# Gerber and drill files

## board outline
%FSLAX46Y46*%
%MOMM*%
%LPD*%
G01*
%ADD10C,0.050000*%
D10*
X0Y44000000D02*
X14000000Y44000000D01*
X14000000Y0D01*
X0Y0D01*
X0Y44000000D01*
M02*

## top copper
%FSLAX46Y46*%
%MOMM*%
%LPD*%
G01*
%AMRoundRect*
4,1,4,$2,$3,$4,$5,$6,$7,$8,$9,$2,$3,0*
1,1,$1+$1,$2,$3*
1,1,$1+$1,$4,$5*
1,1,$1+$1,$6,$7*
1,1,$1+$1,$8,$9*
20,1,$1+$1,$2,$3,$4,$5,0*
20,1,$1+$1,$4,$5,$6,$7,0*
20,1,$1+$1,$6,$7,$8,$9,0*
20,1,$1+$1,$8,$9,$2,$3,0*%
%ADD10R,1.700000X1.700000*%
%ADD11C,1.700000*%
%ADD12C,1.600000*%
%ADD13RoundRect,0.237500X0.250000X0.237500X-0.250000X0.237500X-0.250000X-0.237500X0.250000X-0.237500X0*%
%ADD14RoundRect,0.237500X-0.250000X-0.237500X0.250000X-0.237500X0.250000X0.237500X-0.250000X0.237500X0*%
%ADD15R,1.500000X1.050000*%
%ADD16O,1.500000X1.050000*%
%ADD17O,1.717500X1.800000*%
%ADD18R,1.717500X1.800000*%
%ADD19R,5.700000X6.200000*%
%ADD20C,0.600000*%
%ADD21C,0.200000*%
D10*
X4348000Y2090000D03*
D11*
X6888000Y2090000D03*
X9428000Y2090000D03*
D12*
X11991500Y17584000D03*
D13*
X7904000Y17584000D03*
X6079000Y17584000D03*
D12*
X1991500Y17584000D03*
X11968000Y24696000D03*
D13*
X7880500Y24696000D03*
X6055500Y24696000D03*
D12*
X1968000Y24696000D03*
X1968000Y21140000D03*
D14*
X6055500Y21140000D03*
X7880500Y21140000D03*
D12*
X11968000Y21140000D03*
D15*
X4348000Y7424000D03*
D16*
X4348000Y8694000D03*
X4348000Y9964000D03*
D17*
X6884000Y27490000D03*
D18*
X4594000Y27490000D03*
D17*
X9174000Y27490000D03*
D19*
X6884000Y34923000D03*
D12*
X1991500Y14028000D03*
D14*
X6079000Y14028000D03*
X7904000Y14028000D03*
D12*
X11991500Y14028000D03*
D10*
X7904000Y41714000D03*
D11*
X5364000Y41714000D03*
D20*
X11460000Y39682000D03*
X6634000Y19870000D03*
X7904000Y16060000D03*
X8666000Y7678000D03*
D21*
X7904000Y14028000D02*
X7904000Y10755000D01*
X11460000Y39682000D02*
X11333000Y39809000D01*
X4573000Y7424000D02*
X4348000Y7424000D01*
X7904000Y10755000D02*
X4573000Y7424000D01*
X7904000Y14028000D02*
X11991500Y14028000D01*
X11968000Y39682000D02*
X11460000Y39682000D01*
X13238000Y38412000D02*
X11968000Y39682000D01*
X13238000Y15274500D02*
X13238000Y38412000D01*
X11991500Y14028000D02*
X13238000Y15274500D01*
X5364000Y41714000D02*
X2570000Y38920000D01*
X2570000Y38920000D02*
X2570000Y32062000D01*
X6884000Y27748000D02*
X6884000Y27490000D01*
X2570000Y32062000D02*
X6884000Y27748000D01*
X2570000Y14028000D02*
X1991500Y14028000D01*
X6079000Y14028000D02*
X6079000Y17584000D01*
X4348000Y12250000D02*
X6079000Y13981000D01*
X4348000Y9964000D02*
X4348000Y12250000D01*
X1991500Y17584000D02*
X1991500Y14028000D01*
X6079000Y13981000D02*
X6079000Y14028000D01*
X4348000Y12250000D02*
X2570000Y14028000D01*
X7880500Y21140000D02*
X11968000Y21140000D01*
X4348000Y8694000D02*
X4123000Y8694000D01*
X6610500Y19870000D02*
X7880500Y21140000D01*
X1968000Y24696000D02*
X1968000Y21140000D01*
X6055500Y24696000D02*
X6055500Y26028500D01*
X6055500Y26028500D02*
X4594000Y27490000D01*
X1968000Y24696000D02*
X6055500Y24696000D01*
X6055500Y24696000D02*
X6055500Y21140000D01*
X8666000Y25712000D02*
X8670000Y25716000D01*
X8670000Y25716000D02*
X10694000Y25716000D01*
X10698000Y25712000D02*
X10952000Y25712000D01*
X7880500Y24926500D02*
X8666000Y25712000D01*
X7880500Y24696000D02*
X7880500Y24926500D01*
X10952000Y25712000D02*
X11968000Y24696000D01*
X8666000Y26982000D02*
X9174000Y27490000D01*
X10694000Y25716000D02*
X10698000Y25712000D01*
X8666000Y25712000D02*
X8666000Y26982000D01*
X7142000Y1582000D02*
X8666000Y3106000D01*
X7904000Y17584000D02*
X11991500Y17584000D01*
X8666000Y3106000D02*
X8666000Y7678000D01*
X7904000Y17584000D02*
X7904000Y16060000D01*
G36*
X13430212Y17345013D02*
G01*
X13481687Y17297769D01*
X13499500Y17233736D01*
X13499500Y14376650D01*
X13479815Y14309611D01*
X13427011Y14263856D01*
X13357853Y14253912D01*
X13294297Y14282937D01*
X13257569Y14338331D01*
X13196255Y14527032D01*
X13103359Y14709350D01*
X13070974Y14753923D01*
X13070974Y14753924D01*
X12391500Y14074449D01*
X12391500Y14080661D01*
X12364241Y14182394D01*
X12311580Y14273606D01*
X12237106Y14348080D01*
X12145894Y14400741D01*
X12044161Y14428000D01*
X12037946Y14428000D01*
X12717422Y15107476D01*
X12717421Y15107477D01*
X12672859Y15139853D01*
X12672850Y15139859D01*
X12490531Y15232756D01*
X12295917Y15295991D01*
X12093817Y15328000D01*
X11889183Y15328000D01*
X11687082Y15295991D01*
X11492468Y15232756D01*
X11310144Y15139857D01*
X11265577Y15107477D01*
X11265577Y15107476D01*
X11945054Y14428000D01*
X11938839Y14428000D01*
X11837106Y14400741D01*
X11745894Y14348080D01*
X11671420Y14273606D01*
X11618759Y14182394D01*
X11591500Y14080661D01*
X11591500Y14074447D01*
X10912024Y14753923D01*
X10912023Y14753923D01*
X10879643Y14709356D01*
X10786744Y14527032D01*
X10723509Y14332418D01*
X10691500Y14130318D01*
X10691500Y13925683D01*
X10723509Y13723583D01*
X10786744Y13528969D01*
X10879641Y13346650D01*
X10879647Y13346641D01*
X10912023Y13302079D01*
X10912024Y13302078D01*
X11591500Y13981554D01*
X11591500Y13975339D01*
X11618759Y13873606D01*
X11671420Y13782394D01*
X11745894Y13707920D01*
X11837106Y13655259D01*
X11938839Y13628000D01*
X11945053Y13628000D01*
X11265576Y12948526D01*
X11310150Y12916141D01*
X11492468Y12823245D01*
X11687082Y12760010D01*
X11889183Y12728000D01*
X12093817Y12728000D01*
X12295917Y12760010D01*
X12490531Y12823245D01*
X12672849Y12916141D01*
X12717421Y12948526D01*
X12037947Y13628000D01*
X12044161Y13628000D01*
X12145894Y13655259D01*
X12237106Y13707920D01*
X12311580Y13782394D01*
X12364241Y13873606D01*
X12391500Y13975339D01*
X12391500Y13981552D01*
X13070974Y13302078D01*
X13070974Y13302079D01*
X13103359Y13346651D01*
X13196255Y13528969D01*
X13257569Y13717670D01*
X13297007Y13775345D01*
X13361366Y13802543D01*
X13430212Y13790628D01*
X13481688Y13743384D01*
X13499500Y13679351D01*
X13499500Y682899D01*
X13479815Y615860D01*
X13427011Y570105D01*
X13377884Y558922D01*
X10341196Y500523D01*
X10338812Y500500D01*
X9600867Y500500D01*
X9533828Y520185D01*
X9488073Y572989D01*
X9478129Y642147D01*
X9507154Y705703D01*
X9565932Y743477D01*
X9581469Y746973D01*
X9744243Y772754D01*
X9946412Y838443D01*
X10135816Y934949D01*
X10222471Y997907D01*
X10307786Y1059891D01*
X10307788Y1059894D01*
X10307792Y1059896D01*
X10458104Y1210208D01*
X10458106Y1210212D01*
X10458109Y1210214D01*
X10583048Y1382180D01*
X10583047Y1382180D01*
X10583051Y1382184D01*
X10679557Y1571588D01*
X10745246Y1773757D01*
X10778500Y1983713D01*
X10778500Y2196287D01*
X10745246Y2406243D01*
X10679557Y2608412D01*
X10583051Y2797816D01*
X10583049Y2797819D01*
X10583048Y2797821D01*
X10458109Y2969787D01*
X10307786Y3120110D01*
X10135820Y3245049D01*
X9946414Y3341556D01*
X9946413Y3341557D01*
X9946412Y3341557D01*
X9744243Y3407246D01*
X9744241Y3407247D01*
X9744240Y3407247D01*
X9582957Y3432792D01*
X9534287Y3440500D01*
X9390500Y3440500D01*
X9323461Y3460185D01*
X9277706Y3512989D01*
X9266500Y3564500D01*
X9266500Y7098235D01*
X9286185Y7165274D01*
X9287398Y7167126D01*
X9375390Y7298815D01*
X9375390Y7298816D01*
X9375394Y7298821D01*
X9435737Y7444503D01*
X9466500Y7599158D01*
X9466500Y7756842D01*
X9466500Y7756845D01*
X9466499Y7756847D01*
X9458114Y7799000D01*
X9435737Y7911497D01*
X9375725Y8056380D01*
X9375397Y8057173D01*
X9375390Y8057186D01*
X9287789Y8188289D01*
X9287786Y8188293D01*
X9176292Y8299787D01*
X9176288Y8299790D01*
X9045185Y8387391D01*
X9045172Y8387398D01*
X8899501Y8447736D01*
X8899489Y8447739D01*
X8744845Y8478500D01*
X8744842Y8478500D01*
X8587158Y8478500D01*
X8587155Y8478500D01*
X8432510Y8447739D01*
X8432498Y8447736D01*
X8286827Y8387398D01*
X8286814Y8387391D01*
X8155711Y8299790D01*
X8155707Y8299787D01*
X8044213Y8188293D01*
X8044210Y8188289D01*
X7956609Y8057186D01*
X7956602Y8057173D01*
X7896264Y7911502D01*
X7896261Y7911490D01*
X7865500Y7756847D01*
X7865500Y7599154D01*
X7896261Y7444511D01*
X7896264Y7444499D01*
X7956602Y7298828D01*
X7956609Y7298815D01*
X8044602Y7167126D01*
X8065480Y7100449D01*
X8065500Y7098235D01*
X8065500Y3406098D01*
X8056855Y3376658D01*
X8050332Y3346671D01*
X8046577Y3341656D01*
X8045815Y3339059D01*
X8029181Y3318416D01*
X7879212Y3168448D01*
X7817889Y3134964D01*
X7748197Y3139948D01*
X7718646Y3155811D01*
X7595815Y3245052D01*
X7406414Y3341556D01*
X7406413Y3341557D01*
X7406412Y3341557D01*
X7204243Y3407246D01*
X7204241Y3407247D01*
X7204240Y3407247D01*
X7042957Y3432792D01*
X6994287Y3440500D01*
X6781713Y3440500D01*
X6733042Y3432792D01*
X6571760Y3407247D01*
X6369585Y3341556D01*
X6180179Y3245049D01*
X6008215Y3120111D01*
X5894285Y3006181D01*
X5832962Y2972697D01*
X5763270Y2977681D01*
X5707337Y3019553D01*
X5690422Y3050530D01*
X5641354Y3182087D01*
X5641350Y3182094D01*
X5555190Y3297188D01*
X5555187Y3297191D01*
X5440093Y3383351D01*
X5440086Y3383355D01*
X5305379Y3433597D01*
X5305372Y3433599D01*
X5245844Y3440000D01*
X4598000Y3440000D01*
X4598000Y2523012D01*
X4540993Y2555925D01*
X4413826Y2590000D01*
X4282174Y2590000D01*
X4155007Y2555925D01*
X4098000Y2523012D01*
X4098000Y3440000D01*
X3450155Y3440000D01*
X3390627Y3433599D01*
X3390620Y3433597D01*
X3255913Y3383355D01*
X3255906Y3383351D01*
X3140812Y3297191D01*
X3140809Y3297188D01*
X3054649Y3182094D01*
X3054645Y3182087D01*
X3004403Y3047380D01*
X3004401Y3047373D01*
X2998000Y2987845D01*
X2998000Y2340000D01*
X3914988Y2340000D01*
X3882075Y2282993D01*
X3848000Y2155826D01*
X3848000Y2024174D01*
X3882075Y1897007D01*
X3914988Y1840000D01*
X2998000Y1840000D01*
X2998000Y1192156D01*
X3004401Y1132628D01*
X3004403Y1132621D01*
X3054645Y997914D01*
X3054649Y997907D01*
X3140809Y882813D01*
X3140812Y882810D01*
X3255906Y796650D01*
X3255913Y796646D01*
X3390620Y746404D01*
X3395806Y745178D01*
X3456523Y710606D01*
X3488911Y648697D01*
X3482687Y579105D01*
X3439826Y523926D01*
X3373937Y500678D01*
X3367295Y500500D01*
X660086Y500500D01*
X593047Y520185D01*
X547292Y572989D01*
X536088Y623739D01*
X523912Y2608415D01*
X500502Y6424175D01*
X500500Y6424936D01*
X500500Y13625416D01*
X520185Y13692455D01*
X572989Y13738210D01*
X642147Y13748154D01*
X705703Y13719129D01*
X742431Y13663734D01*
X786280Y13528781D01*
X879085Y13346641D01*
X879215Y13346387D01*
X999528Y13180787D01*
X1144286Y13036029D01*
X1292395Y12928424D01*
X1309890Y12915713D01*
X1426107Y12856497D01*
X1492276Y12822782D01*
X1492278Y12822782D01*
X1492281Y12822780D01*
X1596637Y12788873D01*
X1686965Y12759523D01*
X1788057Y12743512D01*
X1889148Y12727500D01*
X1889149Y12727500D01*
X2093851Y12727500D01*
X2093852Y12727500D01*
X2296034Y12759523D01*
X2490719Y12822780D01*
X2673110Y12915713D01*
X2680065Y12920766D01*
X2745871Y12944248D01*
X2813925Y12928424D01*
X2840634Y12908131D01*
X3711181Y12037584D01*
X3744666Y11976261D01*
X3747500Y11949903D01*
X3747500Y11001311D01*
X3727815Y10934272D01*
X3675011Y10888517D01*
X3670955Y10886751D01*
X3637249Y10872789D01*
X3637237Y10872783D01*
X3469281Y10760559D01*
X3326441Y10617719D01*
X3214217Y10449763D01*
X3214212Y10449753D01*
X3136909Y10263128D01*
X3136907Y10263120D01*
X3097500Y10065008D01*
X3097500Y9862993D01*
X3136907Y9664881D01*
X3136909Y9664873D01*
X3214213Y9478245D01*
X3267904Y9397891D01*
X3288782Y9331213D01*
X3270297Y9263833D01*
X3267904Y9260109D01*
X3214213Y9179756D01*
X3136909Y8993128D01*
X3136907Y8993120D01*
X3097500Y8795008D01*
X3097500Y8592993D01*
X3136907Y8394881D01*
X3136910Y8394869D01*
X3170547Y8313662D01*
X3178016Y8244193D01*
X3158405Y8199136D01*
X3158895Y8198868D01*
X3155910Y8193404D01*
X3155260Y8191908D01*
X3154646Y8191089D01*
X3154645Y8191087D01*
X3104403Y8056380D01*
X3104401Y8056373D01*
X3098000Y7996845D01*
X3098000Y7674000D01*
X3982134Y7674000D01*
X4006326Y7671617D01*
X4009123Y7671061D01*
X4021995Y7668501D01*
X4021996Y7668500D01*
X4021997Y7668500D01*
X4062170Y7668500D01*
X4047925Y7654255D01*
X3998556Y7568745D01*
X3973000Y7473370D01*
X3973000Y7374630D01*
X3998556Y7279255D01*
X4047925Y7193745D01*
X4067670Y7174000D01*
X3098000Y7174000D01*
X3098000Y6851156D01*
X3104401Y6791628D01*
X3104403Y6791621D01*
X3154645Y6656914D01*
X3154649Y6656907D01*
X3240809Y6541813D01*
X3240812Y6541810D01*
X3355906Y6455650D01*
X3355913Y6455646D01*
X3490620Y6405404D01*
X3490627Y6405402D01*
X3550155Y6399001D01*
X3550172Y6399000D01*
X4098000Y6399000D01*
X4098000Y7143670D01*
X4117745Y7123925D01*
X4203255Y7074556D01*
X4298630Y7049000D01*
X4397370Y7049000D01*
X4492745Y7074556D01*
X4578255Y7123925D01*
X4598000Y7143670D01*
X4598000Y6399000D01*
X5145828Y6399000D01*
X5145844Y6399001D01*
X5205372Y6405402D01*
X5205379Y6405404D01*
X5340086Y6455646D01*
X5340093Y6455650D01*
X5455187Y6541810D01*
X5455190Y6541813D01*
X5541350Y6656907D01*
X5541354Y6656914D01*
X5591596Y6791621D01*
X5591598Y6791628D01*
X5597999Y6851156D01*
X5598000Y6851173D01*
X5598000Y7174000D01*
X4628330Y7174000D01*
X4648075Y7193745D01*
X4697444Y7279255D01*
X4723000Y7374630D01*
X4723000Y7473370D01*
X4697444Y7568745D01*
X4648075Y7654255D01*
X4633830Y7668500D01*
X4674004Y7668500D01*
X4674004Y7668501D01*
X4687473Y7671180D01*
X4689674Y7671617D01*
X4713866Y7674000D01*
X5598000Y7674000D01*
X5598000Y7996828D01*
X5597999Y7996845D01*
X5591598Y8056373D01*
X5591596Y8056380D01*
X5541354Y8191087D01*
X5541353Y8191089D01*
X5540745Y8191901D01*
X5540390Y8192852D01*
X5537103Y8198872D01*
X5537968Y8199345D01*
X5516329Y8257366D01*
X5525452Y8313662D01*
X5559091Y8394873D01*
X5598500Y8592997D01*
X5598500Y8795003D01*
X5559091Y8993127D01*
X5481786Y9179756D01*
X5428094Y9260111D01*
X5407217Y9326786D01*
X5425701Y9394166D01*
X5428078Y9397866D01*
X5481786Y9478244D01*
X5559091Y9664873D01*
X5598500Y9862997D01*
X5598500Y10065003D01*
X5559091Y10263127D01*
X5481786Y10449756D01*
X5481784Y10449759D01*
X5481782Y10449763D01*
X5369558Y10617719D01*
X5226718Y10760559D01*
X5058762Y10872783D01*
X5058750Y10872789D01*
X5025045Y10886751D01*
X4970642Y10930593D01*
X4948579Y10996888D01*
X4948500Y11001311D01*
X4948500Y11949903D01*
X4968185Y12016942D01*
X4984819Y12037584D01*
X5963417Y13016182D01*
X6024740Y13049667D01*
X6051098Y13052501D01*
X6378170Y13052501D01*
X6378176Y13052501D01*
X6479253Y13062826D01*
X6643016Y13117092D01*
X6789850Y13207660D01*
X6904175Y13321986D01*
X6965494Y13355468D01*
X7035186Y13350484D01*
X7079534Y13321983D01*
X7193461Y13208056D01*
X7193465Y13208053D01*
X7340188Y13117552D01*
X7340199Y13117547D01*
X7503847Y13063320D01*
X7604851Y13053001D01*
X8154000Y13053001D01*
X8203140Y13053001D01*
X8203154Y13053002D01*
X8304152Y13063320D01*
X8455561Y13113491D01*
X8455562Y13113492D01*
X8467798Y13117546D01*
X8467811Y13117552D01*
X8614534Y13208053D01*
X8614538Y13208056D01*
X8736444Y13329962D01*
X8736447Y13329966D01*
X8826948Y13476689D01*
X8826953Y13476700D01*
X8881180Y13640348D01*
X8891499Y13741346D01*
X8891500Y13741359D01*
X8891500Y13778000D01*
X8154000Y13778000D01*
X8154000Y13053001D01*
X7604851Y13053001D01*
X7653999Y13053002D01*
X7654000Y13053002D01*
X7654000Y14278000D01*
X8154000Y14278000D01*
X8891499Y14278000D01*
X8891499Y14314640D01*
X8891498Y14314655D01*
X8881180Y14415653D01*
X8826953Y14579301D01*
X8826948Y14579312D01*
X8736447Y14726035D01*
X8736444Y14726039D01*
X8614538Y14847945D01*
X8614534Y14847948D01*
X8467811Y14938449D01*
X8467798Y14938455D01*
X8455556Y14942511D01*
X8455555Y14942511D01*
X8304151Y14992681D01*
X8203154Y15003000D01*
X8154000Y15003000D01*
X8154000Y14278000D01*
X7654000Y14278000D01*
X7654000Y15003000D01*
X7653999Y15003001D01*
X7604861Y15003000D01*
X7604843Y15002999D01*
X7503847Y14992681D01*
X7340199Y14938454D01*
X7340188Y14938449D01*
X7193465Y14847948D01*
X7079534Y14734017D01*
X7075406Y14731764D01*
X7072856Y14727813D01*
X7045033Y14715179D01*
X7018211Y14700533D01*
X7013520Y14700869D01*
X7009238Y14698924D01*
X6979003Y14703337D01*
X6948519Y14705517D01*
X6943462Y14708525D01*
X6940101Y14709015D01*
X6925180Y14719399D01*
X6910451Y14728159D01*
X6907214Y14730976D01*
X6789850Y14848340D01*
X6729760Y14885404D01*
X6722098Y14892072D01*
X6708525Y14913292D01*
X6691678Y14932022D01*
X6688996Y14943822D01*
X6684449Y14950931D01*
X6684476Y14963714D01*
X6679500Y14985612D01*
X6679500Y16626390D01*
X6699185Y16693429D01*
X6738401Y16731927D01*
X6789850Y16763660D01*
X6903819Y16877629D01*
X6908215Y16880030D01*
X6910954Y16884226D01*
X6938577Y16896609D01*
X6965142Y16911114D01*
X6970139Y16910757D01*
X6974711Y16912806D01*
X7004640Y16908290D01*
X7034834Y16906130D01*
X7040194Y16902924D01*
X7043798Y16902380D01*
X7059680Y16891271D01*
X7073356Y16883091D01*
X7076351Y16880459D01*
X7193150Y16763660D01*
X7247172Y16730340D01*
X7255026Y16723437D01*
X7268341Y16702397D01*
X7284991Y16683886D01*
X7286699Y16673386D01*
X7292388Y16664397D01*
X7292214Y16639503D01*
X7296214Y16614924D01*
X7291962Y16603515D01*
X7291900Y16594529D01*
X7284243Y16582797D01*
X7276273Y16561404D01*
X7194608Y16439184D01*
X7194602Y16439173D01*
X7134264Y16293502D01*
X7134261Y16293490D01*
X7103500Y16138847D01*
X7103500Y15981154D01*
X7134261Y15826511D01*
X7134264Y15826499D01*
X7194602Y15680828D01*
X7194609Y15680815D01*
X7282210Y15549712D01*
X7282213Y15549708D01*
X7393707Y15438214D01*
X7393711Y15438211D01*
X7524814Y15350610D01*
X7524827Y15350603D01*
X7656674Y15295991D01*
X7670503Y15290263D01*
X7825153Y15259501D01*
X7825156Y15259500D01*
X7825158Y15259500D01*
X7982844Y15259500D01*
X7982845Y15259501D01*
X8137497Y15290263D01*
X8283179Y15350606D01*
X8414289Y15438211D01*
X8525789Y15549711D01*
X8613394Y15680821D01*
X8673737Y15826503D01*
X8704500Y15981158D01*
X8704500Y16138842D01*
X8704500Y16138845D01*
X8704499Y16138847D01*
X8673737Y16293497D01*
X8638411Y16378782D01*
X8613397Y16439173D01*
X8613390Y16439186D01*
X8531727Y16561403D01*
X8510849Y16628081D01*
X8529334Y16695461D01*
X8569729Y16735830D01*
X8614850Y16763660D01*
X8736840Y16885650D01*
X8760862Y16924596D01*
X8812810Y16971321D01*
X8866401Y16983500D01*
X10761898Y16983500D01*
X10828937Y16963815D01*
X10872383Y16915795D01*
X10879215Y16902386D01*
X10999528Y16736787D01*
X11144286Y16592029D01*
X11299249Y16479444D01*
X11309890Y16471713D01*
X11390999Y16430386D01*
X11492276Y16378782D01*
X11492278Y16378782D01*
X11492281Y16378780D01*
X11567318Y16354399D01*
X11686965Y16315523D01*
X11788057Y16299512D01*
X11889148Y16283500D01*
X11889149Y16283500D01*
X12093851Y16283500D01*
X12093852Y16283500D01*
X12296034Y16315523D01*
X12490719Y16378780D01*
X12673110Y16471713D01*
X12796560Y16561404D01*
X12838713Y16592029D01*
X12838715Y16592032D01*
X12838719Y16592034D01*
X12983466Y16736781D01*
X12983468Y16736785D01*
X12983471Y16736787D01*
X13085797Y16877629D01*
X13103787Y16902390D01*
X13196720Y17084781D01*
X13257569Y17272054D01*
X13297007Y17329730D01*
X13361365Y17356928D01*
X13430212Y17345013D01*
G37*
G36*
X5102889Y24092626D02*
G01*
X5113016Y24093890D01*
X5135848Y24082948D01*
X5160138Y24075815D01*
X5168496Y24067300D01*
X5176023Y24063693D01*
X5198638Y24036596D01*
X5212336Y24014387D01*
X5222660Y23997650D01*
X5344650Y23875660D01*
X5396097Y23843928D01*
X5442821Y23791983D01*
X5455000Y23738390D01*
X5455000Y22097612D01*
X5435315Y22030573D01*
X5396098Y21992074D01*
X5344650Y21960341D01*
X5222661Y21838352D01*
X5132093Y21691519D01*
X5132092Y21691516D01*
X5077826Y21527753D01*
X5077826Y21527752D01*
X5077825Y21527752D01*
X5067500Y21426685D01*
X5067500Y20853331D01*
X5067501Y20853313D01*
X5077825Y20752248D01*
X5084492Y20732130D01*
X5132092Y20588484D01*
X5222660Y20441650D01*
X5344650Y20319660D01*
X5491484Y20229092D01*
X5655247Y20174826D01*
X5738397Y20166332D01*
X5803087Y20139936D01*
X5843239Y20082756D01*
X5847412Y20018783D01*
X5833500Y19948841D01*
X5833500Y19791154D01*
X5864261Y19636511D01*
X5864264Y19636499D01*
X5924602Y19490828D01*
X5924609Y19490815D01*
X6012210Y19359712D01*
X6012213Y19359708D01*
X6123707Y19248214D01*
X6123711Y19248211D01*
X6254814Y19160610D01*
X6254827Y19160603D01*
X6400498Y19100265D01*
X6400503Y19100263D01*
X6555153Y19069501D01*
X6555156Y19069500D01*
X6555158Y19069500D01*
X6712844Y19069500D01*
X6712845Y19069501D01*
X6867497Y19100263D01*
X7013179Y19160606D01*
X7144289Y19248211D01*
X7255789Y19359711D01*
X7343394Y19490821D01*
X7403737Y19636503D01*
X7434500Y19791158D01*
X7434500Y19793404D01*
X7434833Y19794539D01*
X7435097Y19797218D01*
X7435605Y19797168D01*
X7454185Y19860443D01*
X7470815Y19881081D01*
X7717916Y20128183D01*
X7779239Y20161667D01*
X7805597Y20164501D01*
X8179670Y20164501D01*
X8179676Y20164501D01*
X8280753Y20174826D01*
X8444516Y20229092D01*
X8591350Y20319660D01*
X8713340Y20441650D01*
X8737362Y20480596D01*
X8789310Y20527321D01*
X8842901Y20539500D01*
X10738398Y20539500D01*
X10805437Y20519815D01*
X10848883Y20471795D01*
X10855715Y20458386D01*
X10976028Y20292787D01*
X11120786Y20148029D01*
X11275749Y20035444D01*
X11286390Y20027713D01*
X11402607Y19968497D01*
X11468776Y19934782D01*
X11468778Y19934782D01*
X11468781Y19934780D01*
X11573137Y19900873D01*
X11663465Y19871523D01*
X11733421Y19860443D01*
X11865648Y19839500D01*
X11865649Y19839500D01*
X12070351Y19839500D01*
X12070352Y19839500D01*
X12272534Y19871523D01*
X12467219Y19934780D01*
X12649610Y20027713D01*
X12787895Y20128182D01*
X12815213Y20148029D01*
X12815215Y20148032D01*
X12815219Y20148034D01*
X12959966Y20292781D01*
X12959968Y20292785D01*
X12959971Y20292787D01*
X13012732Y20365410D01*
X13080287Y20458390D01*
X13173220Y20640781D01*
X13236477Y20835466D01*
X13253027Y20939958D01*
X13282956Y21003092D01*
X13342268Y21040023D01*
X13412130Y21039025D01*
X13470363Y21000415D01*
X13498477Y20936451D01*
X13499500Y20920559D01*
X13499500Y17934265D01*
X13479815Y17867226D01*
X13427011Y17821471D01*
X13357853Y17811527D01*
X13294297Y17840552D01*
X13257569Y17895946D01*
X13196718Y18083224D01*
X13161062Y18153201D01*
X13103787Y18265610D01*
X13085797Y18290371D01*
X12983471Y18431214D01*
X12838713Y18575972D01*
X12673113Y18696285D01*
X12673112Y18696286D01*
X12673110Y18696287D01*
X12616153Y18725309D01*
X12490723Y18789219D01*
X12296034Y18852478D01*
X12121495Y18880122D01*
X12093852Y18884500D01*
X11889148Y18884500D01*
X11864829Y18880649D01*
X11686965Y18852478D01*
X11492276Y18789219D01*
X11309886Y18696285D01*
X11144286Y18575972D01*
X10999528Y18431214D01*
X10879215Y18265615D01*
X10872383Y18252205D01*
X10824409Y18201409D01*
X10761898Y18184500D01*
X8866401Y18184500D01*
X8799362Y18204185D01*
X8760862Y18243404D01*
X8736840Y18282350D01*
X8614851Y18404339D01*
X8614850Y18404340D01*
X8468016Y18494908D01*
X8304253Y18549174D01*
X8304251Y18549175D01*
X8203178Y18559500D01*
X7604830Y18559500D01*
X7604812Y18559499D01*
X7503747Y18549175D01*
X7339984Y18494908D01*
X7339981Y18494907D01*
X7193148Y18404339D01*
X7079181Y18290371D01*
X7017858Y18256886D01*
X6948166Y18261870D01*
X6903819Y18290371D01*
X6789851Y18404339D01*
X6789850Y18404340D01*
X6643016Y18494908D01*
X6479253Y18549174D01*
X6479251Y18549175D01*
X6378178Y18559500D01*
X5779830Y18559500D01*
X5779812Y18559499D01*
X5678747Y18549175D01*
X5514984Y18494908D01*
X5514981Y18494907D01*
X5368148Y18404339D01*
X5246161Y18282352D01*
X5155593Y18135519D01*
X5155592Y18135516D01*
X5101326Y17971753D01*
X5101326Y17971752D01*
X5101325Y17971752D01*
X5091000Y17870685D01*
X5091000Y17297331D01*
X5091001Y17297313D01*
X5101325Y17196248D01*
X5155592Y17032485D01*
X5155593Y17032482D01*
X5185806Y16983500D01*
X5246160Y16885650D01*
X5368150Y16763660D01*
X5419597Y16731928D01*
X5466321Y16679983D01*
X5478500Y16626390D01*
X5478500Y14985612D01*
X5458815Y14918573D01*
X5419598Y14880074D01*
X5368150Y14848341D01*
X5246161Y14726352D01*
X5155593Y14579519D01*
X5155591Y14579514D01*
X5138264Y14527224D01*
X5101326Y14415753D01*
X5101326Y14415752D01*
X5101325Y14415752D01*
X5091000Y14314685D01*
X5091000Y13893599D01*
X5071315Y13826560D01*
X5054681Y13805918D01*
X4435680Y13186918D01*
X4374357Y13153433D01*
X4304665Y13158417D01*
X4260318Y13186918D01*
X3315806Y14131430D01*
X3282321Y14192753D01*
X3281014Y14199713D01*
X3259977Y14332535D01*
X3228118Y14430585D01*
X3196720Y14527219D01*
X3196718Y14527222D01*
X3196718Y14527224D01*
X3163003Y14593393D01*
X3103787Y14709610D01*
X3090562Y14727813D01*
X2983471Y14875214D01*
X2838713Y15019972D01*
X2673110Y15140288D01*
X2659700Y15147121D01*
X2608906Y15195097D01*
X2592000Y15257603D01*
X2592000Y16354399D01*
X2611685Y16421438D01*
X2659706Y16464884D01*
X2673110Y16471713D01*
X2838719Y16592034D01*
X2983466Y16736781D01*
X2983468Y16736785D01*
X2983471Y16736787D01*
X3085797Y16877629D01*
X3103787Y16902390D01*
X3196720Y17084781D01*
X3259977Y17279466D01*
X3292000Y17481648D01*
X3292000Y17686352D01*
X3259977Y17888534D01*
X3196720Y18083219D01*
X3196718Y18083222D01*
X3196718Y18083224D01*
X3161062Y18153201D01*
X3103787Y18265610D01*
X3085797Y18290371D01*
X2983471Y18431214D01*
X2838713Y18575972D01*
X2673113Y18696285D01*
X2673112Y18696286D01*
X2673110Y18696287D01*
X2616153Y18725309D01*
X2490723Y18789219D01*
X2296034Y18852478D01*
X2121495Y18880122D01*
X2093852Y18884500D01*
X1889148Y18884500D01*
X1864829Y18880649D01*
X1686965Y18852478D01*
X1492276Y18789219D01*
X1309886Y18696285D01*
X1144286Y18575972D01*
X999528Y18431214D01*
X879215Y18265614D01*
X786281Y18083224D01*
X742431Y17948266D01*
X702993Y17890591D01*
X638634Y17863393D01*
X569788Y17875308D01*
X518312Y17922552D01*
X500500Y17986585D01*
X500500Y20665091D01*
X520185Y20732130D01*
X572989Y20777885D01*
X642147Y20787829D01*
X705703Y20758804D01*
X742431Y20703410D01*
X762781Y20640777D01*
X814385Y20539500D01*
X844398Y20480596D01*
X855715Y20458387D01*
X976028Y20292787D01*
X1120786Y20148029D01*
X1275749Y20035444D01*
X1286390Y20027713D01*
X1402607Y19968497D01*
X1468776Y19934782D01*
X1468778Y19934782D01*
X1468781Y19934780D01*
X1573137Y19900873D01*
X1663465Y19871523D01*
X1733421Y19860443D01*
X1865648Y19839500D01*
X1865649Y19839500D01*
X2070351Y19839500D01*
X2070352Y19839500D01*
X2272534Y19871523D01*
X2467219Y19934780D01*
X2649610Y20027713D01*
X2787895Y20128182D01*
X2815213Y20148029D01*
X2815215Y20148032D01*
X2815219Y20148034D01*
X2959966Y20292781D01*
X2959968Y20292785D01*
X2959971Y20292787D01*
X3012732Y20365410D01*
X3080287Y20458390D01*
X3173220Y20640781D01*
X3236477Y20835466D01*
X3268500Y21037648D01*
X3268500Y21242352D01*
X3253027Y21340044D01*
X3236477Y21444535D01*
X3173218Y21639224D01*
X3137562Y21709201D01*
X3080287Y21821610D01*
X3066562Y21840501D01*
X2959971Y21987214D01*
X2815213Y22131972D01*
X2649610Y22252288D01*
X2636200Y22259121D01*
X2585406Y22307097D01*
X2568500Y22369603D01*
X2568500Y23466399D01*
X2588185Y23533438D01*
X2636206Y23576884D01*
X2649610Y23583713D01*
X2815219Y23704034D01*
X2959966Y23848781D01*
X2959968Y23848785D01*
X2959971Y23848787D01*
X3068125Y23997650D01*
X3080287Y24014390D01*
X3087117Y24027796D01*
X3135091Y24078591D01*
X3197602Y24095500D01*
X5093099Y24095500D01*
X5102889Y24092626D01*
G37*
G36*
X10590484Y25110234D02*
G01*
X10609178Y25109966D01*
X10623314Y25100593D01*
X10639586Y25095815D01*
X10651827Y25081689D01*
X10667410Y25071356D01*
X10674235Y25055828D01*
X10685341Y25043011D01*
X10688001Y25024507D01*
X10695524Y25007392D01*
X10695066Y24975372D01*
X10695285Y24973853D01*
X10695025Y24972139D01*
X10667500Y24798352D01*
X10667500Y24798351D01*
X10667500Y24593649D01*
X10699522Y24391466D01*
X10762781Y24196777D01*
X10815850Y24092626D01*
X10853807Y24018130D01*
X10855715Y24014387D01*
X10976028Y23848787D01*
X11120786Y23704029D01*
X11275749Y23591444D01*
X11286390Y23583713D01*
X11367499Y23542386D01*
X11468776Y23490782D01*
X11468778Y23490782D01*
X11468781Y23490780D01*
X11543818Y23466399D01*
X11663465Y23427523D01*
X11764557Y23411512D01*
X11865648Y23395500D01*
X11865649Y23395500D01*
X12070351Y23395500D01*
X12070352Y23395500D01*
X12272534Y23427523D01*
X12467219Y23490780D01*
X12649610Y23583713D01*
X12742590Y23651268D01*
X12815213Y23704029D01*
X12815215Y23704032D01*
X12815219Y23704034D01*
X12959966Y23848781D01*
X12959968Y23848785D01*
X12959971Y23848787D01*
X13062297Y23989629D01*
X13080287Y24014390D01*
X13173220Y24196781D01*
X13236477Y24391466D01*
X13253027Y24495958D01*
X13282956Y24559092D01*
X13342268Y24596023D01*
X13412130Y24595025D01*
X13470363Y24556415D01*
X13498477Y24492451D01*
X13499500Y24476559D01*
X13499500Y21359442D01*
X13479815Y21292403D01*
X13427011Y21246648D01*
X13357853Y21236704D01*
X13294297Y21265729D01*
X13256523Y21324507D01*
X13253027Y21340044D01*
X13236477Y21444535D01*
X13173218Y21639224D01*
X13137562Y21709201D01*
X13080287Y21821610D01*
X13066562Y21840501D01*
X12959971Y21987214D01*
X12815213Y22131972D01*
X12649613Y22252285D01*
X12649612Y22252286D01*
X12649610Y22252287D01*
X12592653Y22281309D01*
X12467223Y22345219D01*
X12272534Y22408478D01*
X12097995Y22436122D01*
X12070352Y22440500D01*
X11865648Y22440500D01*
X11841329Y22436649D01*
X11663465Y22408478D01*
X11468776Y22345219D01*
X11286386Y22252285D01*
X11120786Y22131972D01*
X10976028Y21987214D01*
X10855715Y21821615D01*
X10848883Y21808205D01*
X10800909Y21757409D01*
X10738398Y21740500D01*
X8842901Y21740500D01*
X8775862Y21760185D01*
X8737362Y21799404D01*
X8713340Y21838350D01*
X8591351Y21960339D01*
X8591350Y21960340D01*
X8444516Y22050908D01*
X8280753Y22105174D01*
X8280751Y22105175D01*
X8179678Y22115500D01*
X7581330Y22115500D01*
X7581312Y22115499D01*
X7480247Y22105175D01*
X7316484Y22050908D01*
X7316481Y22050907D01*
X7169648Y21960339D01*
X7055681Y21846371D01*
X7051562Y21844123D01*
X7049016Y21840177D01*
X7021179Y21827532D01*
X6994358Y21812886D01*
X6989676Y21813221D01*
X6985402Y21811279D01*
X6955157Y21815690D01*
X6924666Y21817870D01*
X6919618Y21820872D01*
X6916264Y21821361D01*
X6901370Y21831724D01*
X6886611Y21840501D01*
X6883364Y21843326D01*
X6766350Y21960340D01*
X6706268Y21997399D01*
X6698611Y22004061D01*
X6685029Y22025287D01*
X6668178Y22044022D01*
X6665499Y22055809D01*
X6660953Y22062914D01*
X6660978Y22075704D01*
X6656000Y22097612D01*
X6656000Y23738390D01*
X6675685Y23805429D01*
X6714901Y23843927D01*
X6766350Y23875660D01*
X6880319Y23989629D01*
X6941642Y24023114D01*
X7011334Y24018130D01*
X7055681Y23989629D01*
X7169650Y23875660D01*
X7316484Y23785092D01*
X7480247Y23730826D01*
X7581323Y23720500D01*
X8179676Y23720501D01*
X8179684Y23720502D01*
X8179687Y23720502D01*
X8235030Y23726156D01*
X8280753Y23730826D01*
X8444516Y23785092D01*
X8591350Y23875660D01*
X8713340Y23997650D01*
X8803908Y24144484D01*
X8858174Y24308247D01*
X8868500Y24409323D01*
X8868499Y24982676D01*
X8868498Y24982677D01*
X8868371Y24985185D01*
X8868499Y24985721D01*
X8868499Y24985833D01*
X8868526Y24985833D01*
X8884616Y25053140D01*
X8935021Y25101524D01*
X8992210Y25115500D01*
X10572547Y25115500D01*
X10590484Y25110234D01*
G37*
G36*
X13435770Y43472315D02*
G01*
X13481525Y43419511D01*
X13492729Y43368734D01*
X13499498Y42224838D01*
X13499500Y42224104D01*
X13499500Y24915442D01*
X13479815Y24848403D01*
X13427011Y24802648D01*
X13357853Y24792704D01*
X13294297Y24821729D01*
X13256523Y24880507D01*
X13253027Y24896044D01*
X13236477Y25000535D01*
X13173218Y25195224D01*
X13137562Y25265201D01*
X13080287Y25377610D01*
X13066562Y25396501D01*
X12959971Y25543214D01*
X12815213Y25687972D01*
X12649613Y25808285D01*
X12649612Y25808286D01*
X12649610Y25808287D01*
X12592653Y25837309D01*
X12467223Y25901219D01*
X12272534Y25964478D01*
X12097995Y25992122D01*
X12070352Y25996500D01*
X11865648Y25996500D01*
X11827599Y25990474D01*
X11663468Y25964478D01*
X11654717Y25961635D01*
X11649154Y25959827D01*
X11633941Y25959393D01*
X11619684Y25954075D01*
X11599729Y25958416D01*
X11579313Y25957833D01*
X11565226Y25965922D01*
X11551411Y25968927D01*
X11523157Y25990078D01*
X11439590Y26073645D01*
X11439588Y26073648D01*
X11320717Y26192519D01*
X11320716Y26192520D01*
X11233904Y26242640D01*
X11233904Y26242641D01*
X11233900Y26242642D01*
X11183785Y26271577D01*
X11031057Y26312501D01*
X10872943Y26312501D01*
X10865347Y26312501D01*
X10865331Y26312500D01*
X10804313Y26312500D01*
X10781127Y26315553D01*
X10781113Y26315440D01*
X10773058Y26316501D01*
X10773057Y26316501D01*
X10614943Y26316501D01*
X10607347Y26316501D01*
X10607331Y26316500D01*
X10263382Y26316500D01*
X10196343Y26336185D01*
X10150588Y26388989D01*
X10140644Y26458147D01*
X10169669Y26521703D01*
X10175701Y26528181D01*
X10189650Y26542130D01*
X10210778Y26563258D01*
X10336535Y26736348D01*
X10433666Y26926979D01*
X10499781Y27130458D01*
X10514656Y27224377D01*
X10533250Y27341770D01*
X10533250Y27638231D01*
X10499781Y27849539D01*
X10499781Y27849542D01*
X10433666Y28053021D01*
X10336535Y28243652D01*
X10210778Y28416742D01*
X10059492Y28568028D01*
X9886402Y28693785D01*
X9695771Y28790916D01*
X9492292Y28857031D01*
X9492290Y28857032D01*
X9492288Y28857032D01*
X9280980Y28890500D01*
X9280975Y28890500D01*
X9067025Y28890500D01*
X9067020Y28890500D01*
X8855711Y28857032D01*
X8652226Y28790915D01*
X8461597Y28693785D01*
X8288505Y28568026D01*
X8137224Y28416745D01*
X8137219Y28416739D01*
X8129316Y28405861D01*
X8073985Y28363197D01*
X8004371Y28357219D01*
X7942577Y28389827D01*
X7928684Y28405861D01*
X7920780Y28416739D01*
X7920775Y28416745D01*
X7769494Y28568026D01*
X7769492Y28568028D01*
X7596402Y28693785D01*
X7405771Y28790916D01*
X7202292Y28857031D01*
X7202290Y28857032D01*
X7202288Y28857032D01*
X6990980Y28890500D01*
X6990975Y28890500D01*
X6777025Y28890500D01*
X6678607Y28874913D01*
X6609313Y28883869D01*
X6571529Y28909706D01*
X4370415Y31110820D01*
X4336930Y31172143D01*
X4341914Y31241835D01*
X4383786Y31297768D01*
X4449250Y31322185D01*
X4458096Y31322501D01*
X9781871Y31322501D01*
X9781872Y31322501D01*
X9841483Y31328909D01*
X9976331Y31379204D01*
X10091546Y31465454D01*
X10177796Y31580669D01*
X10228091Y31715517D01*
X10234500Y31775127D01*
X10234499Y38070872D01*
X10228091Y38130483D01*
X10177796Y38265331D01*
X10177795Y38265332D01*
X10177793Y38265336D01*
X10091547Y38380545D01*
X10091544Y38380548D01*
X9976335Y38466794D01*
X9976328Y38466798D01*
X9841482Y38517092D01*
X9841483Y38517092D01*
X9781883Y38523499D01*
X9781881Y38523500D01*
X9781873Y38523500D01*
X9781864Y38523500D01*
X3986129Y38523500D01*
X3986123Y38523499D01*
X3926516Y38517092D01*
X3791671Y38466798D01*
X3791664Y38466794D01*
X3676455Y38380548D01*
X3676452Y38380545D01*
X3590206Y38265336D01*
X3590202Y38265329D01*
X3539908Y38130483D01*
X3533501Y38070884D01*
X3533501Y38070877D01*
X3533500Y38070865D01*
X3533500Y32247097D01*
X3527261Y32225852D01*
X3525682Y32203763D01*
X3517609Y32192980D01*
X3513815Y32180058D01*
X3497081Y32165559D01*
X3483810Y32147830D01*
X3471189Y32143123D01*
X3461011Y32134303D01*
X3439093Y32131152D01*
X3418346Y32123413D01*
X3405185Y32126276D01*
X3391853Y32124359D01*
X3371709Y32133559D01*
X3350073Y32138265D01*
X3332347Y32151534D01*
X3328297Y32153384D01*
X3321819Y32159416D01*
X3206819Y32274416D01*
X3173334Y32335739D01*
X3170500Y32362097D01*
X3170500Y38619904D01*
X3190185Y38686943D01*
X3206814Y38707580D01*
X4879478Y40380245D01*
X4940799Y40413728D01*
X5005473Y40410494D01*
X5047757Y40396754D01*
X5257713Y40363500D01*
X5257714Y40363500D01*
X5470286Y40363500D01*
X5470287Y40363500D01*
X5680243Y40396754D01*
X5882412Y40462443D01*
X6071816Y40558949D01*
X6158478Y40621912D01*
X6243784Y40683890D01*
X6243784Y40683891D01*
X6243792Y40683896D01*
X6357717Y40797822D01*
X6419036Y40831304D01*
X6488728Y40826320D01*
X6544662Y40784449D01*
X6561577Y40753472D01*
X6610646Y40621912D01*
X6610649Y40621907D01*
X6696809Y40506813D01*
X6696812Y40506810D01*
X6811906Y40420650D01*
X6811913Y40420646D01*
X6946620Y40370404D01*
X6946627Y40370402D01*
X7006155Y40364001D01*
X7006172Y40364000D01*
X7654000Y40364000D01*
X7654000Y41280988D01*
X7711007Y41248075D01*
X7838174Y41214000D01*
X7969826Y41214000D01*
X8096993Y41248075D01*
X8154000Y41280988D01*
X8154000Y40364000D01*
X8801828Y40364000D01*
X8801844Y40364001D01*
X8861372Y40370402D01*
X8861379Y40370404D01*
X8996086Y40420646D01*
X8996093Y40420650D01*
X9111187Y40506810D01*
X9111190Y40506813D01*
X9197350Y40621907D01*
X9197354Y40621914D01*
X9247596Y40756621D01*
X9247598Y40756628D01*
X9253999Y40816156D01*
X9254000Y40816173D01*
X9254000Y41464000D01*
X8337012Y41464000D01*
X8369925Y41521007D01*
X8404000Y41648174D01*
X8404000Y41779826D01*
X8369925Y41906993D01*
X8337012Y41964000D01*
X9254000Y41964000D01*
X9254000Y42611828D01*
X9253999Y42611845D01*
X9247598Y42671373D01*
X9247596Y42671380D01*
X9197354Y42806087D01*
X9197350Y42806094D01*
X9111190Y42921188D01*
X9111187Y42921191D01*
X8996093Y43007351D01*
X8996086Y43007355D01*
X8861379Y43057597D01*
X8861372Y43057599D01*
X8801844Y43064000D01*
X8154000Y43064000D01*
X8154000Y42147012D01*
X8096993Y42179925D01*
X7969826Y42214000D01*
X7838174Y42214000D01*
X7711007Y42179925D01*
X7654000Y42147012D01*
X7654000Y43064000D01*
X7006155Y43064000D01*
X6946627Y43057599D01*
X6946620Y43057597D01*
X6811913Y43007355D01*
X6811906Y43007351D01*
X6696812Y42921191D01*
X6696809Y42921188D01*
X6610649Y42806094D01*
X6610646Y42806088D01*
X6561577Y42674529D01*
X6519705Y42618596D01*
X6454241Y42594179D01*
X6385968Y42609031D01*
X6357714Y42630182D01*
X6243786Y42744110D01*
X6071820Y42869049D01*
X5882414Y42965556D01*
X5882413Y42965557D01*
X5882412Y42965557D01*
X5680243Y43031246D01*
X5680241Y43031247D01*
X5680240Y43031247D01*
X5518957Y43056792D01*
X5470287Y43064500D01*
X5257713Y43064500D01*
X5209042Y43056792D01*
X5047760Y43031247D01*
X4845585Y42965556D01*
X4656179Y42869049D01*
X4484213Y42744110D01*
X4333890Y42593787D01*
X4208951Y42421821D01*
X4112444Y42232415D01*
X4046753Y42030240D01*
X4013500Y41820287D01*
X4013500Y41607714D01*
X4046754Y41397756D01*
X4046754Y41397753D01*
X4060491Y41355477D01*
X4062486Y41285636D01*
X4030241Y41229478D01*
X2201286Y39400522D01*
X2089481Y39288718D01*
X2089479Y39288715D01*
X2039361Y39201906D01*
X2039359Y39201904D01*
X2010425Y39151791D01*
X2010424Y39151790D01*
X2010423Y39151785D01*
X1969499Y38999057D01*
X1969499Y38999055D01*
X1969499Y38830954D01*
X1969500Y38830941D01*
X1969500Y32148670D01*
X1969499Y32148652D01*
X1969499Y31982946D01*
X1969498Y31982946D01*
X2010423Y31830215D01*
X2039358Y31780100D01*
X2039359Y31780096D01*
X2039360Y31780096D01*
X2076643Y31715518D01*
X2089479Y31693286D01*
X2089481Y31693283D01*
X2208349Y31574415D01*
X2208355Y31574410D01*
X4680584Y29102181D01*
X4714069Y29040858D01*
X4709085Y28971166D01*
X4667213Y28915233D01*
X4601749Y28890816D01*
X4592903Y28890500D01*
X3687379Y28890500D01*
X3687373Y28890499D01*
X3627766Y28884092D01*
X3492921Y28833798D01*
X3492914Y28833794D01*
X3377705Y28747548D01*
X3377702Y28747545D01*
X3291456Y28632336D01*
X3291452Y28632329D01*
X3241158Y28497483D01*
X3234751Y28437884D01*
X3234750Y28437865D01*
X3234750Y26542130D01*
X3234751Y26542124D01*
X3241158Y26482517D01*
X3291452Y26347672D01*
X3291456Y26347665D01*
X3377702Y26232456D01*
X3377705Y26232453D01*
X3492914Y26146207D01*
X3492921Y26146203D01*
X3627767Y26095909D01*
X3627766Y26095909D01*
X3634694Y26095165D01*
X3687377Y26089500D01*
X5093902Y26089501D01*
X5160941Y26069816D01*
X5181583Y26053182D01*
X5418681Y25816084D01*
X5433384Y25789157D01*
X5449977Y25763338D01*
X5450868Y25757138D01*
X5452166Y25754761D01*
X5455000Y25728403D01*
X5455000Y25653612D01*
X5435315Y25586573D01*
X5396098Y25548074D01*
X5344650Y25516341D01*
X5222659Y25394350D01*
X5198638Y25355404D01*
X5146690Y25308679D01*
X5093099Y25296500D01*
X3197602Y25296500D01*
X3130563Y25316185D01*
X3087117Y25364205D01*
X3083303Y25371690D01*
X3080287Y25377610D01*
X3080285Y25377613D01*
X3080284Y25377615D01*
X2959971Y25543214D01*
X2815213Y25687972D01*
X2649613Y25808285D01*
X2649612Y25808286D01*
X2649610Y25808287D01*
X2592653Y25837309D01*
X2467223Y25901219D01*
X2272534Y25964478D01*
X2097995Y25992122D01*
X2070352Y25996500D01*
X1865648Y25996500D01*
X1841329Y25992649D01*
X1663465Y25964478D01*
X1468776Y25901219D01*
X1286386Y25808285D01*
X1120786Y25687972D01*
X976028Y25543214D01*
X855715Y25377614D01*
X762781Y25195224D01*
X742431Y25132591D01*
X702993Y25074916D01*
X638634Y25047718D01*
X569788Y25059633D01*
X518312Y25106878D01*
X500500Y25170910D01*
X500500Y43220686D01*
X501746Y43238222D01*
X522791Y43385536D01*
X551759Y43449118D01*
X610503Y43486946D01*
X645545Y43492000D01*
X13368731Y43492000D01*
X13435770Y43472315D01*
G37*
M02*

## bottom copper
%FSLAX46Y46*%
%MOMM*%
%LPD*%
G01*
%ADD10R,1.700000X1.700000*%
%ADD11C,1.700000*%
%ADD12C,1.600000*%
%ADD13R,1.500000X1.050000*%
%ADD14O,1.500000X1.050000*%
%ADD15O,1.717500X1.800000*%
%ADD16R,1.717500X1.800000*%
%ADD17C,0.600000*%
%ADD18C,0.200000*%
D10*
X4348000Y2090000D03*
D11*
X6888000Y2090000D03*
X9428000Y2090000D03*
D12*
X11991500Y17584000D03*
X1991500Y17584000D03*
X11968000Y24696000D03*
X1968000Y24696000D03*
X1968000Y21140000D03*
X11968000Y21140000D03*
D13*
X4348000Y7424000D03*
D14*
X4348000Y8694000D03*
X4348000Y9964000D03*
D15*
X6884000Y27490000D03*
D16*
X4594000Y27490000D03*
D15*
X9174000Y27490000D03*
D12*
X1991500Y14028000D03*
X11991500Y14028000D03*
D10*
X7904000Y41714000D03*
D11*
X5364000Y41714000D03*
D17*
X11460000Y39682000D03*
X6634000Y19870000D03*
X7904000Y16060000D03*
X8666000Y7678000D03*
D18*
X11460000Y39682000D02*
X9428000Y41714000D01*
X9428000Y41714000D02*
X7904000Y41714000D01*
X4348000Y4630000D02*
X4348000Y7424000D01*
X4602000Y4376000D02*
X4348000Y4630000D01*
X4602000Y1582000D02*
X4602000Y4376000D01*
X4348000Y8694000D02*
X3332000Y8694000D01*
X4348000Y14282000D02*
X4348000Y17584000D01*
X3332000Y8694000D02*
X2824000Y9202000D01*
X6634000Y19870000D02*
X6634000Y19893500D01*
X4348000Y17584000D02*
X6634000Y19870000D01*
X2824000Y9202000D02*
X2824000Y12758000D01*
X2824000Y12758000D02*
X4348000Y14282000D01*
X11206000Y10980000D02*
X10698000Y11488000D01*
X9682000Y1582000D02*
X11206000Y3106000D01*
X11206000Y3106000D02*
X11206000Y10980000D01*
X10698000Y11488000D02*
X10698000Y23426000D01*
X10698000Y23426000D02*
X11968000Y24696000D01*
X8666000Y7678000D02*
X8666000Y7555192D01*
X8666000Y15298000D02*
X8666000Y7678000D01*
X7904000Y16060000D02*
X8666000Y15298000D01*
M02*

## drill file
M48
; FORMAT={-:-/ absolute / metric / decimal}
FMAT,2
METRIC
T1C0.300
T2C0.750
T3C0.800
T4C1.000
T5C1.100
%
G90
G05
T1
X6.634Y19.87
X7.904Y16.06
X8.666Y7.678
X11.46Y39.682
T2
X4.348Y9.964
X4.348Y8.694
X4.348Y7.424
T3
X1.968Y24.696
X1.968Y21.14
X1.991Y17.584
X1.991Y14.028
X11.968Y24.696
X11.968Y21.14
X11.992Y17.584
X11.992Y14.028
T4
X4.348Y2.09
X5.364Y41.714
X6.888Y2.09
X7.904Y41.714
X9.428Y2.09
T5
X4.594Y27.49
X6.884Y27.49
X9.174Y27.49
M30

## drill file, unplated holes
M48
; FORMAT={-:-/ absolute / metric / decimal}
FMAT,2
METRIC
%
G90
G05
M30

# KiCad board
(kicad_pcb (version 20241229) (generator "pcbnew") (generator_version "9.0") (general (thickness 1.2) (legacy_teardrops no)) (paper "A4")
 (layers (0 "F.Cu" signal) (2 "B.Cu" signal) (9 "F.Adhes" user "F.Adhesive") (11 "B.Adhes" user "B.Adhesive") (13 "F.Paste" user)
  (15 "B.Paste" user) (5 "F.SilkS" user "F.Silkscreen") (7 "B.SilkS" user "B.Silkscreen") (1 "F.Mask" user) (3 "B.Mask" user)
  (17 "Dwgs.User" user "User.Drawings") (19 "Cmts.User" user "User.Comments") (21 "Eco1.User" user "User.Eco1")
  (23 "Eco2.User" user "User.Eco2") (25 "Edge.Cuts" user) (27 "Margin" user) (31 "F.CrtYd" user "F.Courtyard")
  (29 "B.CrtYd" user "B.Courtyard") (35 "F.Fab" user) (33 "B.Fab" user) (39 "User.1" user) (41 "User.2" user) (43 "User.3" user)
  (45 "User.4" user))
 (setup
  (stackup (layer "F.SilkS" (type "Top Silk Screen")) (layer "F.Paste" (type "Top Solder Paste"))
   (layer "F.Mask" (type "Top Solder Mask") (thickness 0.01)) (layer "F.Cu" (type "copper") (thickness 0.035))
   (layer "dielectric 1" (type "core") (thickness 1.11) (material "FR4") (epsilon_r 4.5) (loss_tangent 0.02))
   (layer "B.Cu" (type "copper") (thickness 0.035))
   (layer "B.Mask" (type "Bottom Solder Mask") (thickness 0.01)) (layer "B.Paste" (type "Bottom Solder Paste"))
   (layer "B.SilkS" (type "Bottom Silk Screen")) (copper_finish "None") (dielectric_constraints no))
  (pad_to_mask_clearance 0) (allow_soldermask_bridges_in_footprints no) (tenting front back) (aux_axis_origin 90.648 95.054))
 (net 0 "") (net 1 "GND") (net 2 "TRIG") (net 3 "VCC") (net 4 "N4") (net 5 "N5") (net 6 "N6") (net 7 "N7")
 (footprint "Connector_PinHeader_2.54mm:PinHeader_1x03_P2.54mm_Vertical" (layer "F.Cu") (at 94.996 92.964 90)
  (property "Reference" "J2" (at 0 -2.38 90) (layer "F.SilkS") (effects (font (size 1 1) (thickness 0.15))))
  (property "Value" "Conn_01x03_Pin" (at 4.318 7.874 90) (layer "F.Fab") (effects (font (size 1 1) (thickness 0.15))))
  (pad "1" thru_hole rect (at 0 0 90) (size 1.7 1.7) (drill 1) (layers "*.Cu" "*.Mask") (remove_unused_layers no) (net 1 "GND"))
  (pad "2" thru_hole circle (at 0 2.54 90) (size 1.7 1.7) (drill 1) (layers "*.Cu" "*.Mask") (remove_unused_layers no) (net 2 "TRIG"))
  (pad "3" thru_hole circle (at 0 5.08 90) (size 1.7 1.7) (drill 1) (layers "*.Cu" "*.Mask") (remove_unused_layers no) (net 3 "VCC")))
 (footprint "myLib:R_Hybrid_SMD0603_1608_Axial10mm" (layer "F.Cu") (at 97.6395 77.47 180)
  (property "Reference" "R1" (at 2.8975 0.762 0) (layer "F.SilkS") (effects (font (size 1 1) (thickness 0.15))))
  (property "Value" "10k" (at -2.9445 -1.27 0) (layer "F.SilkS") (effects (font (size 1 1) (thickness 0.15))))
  (pad "1" thru_hole circle (at -5 0 180) (size 1.6 1.6) (drill 0.8) (layers "*.Cu" "*.Mask") (remove_unused_layers no) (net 2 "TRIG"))
  (pad "1" smd roundrect (at -0.9125 0 180) (size 0.975 0.95) (layers "F.Cu" "F.Mask" "F.Paste") (roundrect_rratio 0.25) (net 2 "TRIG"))
  (pad "2" smd roundrect (at 0.9125 0 180) (size 0.975 0.95) (layers "F.Cu" "F.Mask" "F.Paste") (roundrect_rratio 0.25) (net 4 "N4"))
  (pad "2" thru_hole circle (at 5 0 180) (size 1.6 1.6) (drill 0.8) (layers "*.Cu" "*.Mask") (remove_unused_layers no) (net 4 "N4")))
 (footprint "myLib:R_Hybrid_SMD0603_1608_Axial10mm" (layer "F.Cu") (at 97.616 70.358 180)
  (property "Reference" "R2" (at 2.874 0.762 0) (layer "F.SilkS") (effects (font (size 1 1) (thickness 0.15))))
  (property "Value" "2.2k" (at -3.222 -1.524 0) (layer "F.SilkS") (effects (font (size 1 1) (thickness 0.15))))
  (pad "1" thru_hole circle (at -5 0 180) (size 1.6 1.6) (drill 0.8) (layers "*.Cu" "*.Mask") (remove_unused_layers no) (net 3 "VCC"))
  (pad "1" smd roundrect (at -0.9125 0 180) (size 0.975 0.95) (layers "F.Cu" "F.Mask" "F.Paste") (roundrect_rratio 0.25) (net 3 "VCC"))
  (pad "2" smd roundrect (at 0.9125 0 180) (size 0.975 0.95) (layers "F.Cu" "F.Mask" "F.Paste") (roundrect_rratio 0.25) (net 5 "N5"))
  (pad "2" thru_hole circle (at 5 0 180) (size 1.6 1.6) (drill 0.8) (layers "*.Cu" "*.Mask") (remove_unused_layers no) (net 5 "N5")))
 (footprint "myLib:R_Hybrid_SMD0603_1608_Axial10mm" (layer "F.Cu") (at 97.616 73.914)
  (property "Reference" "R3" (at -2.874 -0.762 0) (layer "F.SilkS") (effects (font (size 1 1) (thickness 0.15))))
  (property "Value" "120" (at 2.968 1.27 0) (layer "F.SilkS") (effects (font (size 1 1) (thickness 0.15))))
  (pad "1" thru_hole circle (at -5 0) (size 1.6 1.6) (drill 0.8) (layers "*.Cu" "*.Mask") (remove_unused_layers no) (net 5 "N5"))
  (pad "1" smd roundrect (at -0.9125 0) (size 0.975 0.95) (layers "F.Cu" "F.Mask" "F.Paste") (roundrect_rratio 0.25) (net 5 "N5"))
  (pad "2" smd roundrect (at 0.9125 0) (size 0.975 0.95) (layers "F.Cu" "F.Mask" "F.Paste") (roundrect_rratio 0.25) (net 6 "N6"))
  (pad "2" thru_hole circle (at 5 0) (size 1.6 1.6) (drill 0.8) (layers "*.Cu" "*.Mask") (remove_unused_layers no) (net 6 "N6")))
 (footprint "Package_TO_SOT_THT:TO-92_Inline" (layer "F.Cu") (at 94.996 87.63 90)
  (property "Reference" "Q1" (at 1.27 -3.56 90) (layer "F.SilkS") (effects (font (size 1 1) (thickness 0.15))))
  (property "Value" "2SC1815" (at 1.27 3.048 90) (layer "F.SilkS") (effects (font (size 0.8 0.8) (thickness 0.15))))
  (pad "1" thru_hole rect (at 0 0 90) (size 1.05 1.5) (drill 0.75) (layers "*.Cu" "*.Mask") (remove_unused_layers no) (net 1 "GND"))
  (pad "2" thru_hole oval (at 1.27 0 90) (size 1.05 1.5) (drill 0.75) (layers "*.Cu" "*.Mask") (remove_unused_layers no) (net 6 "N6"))
  (pad "3" thru_hole oval (at 2.54 0 90) (size 1.05 1.5) (drill 0.75) (layers "*.Cu" "*.Mask") (remove_unused_layers no) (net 4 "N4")))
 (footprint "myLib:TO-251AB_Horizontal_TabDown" (layer "F.Cu") (at 95.242 67.564)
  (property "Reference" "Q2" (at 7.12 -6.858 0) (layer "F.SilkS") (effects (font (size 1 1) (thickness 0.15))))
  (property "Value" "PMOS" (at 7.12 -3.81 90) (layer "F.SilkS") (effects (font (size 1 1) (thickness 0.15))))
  (pad "1" thru_hole oval (at 2.29 0) (size 1.7175 1.8) (drill 1.1) (layers "*.Cu" "*.Mask") (remove_unused_layers no) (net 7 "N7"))
  (pad "2" thru_hole rect (at 0 0) (size 1.7175 1.8) (drill 1.1) (layers "*.Cu" "*.Mask") (remove_unused_layers no) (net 5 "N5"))
  (pad "3" thru_hole oval (at 4.58 0) (size 1.7175 1.8) (drill 1.1) (layers "*.Cu" "*.Mask") (remove_unused_layers no) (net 3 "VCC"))
  (pad "4" smd rect (at 2.29 -7.433) (size 5.7 6.2) (layers "F.Cu" "F.Mask" "F.Paste")))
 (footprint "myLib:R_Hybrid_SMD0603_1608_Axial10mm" (layer "F.Cu") (at 97.6395 81.026)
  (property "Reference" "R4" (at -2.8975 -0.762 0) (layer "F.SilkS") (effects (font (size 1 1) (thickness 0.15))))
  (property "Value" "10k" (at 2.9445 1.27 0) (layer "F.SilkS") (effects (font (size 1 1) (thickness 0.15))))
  (pad "1" thru_hole circle (at -5 0) (size 1.6 1.6) (drill 0.8) (layers "*.Cu" "*.Mask") (remove_unused_layers no) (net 4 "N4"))
  (pad "1" smd roundrect (at -0.9125 0) (size 0.975 0.95) (layers "F.Cu" "F.Mask" "F.Paste") (roundrect_rratio 0.25) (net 4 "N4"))
  (pad "2" smd roundrect (at 0.9125 0) (size 0.975 0.95) (layers "F.Cu" "F.Mask" "F.Paste") (roundrect_rratio 0.25) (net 1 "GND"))
  (pad "2" thru_hole circle (at 5 0) (size 1.6 1.6) (drill 0.8) (layers "*.Cu" "*.Mask") (remove_unused_layers no) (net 1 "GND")))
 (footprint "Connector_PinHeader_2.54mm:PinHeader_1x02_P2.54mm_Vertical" (layer "F.Cu") (at 98.552 53.34 -90)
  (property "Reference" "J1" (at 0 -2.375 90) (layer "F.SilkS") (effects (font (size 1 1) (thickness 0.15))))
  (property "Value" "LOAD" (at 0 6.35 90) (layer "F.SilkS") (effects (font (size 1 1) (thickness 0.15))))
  (pad "1" thru_hole rect (at 0 0 270) (size 1.7 1.7) (drill 1) (layers "*.Cu" "*.Mask") (remove_unused_layers no) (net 1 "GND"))
  (pad "2" thru_hole circle (at 0 2.54 270) (size 1.7 1.7) (drill 1) (layers "*.Cu" "*.Mask") (remove_unused_layers no) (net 7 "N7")))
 (gr_rect (start 90.648 51.054) (end 104.648 95.054) (stroke (width 0.05) (type solid)) (fill no) (layer "Edge.Cuts"))
 (segment (start 98.552 81.026) (end 98.552 84.299) (width 0.2) (layer "F.Cu") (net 1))
 (segment (start 102.108 55.372) (end 101.981 55.245) (width 0.2) (layer "F.Cu") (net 1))
 (segment (start 95.221 87.63) (end 94.996 87.63) (width 0.2) (layer "F.Cu") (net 1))
 (segment (start 98.552 84.299) (end 95.221 87.63) (width 0.2) (layer "F.Cu") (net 1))
 (segment (start 98.552 81.026) (end 102.6395 81.026) (width 0.2) (layer "F.Cu") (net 1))
 (segment (start 102.616 55.372) (end 102.108 55.372) (width 0.2) (layer "F.Cu") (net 1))
 (segment (start 103.886 56.642) (end 102.616 55.372) (width 0.2) (layer "F.Cu") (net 1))
 (segment (start 103.886 79.7795) (end 103.886 56.642) (width 0.2) (layer "F.Cu") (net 1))
 (segment (start 102.6395 81.026) (end 103.886 79.7795) (width 0.2) (layer "F.Cu") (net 1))
 (via (at 102.108 55.372) (size 0.6) (drill 0.3) (layers "F.Cu" "B.Cu") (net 1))
 (segment (start 102.108 55.372) (end 100.076 53.34) (width 0.2) (layer "B.Cu") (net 1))
 (segment (start 100.076 53.34) (end 98.552 53.34) (width 0.2) (layer "B.Cu") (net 1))
 (segment (start 94.996 90.424) (end 94.996 87.63) (width 0.2) (layer "B.Cu") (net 1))
 (segment (start 95.25 90.678) (end 94.996 90.424) (width 0.2) (layer "B.Cu") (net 1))
 (segment (start 95.25 93.472) (end 95.25 90.678) (width 0.2) (layer "B.Cu") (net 1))
 (segment (start 96.012 53.34) (end 93.218 56.134) (width 0.2) (layer "F.Cu") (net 7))
 (segment (start 93.218 56.134) (end 93.218 62.992) (width 0.2) (layer "F.Cu") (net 7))
 (segment (start 97.532 67.306) (end 97.532 67.564) (width 0.2) (layer "F.Cu") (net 7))
 (segment (start 93.218 62.992) (end 97.532 67.306) (width 0.2) (layer "F.Cu") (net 7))
 (segment (start 93.218 81.026) (end 92.6395 81.026) (width 0.2) (layer "F.Cu") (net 4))
 (segment (start 96.727 81.026) (end 96.727 77.47) (width 0.2) (layer "F.Cu") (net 4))
 (segment (start 94.996 82.804) (end 96.727 81.073) (width 0.2) (layer "F.Cu") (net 4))
 (segment (start 94.996 85.09) (end 94.996 82.804) (width 0.2) (layer "F.Cu") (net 4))
 (segment (start 92.6395 77.47) (end 92.6395 81.026) (width 0.2) (layer "F.Cu") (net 4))
 (segment (start 96.727 81.073) (end 96.727 81.026) (width 0.2) (layer "F.Cu") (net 4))
 (segment (start 94.996 82.804) (end 93.218 81.026) (width 0.2) (layer "F.Cu") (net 4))
 (segment (start 98.5285 73.914) (end 102.616 73.914) (width 0.2) (layer "F.Cu") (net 6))
 (segment (start 94.996 86.36) (end 94.771 86.36) (width 0.2) (layer "F.Cu") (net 6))
 (segment (start 97.2585 75.184) (end 98.5285 73.914) (width 0.2) (layer "F.Cu") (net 6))
 (via (at 97.282 75.184) (size 0.6) (drill 0.3) (layers "F.Cu" "B.Cu") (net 6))
 (segment (start 94.996 86.36) (end 93.98 86.36) (width 0.2) (layer "B.Cu") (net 6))
 (segment (start 94.996 80.772) (end 94.996 77.47) (width 0.2) (layer "B.Cu") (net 6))
 (segment (start 93.98 86.36) (end 93.472 85.852) (width 0.2) (layer "B.Cu") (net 6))
 (segment (start 97.282 75.184) (end 97.282 75.1605) (width 0.2) (layer "B.Cu") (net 6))
 (segment (start 94.996 77.47) (end 97.282 75.184) (width 0.2) (layer "B.Cu") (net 6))
 (segment (start 93.472 85.852) (end 93.472 82.296) (width 0.2) (layer "B.Cu") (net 6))
 (segment (start 93.472 82.296) (end 94.996 80.772) (width 0.2) (layer "B.Cu") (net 6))
 (segment (start 92.616 70.358) (end 92.616 73.914) (width 0.2) (layer "F.Cu") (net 5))
 (segment (start 96.7035 70.358) (end 96.7035 69.0255) (width 0.2) (layer "F.Cu") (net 5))
 (segment (start 96.7035 69.0255) (end 95.242 67.564) (width 0.2) (layer "F.Cu") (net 5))
 (segment (start 92.616 70.358) (end 96.7035 70.358) (width 0.2) (layer "F.Cu") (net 5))
 (segment (start 96.7035 70.358) (end 96.7035 73.914) (width 0.2) (layer "F.Cu") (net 5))
 (segment (start 99.314 69.342) (end 99.318 69.338) (width 0.2) (layer "F.Cu") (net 3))
 (segment (start 99.318 69.338) (end 101.342 69.338) (width 0.2) (layer "F.Cu") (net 3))
 (segment (start 101.346 69.342) (end 101.6 69.342) (width 0.2) (layer "F.Cu") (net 3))
 (segment (start 98.5285 70.1275) (end 99.314 69.342) (width 0.2) (layer "F.Cu") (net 3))
 (segment (start 98.5285 70.358) (end 98.5285 70.1275) (width 0.2) (layer "F.Cu") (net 3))
 (segment (start 101.6 69.342) (end 102.616 70.358) (width 0.2) (layer "F.Cu") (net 3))
 (segment (start 99.314 68.072) (end 99.822 67.564) (width 0.2) (layer "F.Cu") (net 3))
 (segment (start 101.342 69.338) (end 101.346 69.342) (width 0.2) (layer "F.Cu") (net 3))
 (segment (start 99.314 69.342) (end 99.314 68.072) (width 0.2) (layer "F.Cu") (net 3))
 (segment (start 101.854 84.074) (end 101.346 83.566) (width 0.2) (layer "B.Cu") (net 3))
 (segment (start 100.33 93.472) (end 101.854 91.948) (width 0.2) (layer "B.Cu") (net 3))
 (segment (start 101.854 91.948) (end 101.854 84.074) (width 0.2) (layer "B.Cu") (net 3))
 (segment (start 101.346 83.566) (end 101.346 71.628) (width 0.2) (layer "B.Cu") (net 3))
 (segment (start 101.346 71.628) (end 102.616 70.358) (width 0.2) (layer "B.Cu") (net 3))
 (segment (start 97.79 93.472) (end 99.314 91.948) (width 0.2) (layer "F.Cu") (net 2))
 (segment (start 98.552 77.47) (end 102.6395 77.47) (width 0.2) (layer "F.Cu") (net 2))
 (segment (start 99.314 91.948) (end 99.314 87.376) (width 0.2) (layer "F.Cu") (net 2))
 (segment (start 98.552 77.47) (end 98.552 78.994) (width 0.2) (layer "F.Cu") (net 2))
 (via (at 98.552 78.994) (size 0.6) (drill 0.3) (layers "F.Cu" "B.Cu") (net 2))
 (via (at 99.314 87.376) (size 0.6) (drill 0.3) (layers "F.Cu" "B.Cu") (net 2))
 (segment (start 99.314 87.376) (end 99.314 87.498808) (width 0.2) (layer "B.Cu") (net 2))
 (segment (start 99.314 79.756) (end 99.314 87.376) (width 0.2) (layer "B.Cu") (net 2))
 (segment (start 98.552 78.994) (end 99.314 79.756) (width 0.2) (layer "B.Cu") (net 2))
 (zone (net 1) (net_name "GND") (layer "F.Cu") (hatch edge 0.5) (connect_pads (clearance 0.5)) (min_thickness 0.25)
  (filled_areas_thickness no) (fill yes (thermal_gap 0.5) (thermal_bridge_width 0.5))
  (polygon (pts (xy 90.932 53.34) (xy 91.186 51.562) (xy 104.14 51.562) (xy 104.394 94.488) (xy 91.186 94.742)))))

